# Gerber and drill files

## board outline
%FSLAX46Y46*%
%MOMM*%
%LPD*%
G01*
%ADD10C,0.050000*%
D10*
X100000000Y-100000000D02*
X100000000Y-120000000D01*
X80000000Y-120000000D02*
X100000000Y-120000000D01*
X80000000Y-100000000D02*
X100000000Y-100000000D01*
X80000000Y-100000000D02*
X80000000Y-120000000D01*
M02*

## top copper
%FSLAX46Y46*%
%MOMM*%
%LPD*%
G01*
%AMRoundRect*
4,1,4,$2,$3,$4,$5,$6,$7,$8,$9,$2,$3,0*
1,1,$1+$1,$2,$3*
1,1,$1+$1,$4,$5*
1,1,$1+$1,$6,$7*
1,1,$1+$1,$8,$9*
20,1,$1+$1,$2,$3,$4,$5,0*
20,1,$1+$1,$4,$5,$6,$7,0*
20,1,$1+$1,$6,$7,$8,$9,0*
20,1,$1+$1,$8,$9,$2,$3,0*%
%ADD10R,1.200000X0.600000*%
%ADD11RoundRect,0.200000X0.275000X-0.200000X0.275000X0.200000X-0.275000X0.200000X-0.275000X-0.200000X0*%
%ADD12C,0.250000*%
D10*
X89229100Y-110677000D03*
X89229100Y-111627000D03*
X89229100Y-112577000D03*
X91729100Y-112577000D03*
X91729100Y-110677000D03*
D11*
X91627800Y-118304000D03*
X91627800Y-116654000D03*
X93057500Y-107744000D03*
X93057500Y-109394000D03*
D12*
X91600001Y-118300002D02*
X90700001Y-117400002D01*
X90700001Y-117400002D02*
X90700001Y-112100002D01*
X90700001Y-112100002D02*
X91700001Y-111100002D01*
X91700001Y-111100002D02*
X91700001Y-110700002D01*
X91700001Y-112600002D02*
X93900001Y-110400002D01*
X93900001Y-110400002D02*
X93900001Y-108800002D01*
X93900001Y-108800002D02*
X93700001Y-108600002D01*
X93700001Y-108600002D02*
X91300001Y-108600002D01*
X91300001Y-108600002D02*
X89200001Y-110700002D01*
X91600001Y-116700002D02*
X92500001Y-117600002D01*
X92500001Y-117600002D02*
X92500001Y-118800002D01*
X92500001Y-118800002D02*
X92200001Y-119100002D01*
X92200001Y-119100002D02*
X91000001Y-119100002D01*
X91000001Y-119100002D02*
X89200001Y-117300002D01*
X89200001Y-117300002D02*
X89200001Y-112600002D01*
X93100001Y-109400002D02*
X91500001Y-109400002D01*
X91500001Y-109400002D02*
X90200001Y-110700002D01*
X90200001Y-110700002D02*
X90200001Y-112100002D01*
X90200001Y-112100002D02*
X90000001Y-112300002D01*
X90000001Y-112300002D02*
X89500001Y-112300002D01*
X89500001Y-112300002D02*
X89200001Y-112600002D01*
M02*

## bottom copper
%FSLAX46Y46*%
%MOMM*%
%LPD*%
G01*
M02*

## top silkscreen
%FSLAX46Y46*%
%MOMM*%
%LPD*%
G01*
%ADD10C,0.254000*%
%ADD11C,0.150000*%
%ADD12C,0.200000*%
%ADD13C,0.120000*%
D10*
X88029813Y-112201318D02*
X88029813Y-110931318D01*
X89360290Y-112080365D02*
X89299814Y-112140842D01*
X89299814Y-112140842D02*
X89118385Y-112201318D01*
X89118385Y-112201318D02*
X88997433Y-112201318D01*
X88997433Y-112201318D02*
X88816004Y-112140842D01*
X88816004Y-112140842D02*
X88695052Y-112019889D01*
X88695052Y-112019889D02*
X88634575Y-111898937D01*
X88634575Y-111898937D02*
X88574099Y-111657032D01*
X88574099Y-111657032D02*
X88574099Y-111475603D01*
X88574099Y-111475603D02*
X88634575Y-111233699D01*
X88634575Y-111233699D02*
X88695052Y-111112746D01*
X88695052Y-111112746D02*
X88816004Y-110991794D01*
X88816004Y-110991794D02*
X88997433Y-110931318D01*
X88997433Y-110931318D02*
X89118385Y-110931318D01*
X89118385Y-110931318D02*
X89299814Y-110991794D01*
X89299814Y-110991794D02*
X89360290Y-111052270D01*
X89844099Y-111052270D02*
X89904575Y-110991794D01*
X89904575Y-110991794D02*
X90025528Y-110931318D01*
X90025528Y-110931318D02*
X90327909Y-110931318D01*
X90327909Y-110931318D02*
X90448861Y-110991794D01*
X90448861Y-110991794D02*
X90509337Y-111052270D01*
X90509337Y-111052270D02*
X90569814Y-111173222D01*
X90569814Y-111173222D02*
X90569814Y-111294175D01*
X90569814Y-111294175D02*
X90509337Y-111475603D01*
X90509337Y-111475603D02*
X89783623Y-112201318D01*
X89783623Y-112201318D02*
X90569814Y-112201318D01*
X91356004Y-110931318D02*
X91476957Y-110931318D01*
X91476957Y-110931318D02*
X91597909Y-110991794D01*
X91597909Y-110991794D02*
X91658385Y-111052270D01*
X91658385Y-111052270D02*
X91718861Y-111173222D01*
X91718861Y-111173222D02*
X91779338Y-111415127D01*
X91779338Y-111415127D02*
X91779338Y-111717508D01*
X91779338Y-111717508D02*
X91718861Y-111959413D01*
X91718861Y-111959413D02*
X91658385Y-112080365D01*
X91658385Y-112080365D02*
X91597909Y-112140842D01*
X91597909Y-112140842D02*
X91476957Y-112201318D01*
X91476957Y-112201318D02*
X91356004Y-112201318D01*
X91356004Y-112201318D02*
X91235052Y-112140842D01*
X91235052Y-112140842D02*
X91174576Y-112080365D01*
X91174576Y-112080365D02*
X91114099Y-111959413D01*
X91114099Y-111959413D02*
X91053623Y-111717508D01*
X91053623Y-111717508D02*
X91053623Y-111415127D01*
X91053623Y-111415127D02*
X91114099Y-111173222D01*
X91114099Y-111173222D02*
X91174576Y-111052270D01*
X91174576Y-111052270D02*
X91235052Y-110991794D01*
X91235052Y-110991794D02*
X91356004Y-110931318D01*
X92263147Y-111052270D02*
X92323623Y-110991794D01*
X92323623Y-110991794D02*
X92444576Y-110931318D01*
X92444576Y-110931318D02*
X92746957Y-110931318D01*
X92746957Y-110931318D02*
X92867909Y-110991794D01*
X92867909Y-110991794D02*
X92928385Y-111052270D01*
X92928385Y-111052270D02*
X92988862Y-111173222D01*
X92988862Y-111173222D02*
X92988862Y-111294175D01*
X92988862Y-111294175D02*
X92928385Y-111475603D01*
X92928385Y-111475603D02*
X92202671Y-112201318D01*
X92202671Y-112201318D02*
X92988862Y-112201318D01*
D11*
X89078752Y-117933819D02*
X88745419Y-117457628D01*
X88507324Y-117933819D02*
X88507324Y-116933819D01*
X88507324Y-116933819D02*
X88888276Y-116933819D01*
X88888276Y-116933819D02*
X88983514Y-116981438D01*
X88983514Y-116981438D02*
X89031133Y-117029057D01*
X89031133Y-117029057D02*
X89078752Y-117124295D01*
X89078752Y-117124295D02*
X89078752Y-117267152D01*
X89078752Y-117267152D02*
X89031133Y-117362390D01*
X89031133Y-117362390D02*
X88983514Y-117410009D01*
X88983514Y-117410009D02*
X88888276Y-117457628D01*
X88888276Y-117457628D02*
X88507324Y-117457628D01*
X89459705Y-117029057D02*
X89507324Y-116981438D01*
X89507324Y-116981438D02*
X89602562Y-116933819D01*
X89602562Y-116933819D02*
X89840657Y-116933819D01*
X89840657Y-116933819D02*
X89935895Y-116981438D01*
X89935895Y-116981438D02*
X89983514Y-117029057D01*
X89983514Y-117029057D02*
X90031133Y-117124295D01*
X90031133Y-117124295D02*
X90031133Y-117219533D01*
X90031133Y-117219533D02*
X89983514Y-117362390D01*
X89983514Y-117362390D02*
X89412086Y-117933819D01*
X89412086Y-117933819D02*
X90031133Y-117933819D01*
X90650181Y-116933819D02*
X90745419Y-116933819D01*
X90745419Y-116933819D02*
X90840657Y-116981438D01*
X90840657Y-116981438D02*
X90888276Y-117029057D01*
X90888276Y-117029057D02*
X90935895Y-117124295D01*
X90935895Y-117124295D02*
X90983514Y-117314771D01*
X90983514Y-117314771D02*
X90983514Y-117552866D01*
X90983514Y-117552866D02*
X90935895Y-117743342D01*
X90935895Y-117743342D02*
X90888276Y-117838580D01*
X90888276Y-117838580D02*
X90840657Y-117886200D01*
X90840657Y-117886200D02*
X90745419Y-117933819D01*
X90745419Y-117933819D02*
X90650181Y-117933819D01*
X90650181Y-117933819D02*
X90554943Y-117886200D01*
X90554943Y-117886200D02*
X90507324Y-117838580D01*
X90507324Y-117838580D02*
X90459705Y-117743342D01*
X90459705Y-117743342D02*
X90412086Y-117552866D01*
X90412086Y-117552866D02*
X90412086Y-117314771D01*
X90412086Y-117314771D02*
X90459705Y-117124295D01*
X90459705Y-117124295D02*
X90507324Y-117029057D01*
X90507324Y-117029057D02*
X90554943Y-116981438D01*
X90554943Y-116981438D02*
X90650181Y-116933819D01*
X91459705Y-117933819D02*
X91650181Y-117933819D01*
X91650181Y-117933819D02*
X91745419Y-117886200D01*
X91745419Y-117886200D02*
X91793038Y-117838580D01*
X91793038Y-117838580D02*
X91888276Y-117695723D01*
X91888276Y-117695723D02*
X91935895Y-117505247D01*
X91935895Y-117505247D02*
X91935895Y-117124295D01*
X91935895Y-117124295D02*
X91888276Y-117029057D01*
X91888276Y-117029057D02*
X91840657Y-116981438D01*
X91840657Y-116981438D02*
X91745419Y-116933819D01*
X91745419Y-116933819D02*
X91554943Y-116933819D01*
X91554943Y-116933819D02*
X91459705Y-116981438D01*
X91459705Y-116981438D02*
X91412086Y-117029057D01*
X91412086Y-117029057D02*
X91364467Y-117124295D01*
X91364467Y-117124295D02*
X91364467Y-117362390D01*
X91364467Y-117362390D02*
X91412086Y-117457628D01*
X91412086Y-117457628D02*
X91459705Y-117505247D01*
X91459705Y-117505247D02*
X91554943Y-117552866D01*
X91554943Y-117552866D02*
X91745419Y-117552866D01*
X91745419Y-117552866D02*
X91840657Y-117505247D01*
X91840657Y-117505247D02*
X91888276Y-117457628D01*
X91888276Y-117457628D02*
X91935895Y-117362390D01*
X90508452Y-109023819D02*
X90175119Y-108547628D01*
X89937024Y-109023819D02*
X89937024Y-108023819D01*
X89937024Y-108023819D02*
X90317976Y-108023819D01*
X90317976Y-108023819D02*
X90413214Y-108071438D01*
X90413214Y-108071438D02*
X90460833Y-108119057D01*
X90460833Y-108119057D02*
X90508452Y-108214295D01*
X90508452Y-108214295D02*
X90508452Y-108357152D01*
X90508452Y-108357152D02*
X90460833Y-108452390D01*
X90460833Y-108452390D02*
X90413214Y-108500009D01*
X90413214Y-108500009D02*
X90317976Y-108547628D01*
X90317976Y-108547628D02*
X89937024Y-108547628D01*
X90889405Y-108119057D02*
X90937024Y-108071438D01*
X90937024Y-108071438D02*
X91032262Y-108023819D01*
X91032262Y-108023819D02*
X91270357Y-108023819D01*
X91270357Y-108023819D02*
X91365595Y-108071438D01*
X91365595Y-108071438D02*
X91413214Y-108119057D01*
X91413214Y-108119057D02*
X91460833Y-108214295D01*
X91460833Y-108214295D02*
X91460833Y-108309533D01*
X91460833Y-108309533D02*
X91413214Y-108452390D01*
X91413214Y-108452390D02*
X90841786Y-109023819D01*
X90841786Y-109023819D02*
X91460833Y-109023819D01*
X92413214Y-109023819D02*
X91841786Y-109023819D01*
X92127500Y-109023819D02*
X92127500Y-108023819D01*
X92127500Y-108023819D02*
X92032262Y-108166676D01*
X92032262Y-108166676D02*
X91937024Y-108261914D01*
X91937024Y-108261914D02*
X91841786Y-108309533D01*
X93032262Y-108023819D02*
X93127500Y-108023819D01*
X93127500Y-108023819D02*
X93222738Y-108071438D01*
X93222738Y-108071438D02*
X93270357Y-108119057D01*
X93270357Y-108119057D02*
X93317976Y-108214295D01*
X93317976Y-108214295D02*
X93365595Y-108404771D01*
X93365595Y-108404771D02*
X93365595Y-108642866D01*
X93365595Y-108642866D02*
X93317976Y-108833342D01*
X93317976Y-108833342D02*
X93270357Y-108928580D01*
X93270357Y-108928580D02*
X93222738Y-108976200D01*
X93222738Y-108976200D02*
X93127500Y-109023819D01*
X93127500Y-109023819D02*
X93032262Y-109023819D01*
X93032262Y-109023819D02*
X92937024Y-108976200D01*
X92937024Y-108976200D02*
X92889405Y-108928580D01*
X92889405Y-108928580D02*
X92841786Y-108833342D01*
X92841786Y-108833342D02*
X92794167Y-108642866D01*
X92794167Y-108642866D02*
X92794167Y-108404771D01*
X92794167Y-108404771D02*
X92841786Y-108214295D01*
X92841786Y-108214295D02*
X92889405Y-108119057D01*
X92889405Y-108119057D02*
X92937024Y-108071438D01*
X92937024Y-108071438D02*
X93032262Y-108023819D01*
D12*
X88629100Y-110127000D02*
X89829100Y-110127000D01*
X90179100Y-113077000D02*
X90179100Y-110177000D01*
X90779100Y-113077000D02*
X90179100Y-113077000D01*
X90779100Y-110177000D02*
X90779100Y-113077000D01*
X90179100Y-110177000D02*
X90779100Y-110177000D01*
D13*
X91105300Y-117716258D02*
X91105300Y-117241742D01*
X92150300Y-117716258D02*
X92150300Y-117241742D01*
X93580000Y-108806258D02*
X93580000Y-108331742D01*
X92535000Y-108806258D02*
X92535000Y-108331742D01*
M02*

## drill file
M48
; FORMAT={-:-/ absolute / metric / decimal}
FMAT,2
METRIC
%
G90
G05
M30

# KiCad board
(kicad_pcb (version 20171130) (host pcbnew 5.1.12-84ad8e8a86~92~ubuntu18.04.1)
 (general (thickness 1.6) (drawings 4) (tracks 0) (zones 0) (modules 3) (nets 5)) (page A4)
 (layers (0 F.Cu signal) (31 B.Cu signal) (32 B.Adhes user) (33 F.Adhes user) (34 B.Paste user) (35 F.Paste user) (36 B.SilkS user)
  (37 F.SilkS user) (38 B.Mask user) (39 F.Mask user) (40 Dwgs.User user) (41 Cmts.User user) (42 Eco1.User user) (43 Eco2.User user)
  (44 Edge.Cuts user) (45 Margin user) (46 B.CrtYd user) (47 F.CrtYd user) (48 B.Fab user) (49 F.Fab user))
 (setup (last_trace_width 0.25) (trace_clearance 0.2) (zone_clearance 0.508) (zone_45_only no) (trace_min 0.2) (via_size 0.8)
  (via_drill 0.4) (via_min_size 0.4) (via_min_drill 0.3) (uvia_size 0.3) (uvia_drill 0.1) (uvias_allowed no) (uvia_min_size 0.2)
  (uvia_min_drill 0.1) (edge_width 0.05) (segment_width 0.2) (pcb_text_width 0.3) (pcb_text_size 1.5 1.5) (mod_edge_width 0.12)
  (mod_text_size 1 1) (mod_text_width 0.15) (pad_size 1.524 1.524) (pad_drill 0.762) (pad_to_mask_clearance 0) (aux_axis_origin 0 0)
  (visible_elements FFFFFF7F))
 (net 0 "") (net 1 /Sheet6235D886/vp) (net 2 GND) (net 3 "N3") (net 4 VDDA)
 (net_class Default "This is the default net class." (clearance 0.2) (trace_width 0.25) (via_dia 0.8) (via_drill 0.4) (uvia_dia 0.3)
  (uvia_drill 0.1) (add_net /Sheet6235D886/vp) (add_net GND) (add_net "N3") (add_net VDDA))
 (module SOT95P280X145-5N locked (layer F.Cu) (at 90.479100 111.627000)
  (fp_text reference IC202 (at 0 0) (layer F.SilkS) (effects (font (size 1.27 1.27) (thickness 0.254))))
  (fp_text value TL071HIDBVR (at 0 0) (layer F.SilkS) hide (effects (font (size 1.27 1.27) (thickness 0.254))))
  (fp_line (start -1.85 -1.5) (end -0.65 -1.5) (layer F.SilkS) (width 0.2))
  (fp_line (start -0.3 1.45) (end -0.3 -1.45) (layer F.SilkS) (width 0.2))
  (fp_line (start 0.3 1.45) (end -0.3 1.45) (layer F.SilkS) (width 0.2))
  (fp_line (start 0.3 -1.45) (end 0.3 1.45) (layer F.SilkS) (width 0.2))
  (fp_line (start -0.3 -1.45) (end 0.3 -1.45) (layer F.SilkS) (width 0.2))
  (pad 1 smd rect (at -1.25 -0.95 90.000000) (size 0.6 1.2) (layers F.Cu F.Mask F.Paste) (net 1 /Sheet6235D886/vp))
  (pad 2 smd rect (at -1.25 0 90.000000) (size 0.6 1.2) (layers F.Cu F.Mask F.Paste) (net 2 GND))
  (pad 3 smd rect (at -1.25 0.95 90.000000) (size 0.6 1.2) (layers F.Cu F.Mask F.Paste) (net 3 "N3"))
  (pad 4 smd rect (at 1.25 0.95 90.000000) (size 0.6 1.2) (layers F.Cu F.Mask F.Paste) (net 1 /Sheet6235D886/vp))
  (pad 5 smd rect (at 1.25 -0.95 90.000000) (size 0.6 1.2) (layers F.Cu F.Mask F.Paste) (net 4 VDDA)))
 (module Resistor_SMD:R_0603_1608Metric (layer F.Cu) (at 91.627800 117.479000 90.000000)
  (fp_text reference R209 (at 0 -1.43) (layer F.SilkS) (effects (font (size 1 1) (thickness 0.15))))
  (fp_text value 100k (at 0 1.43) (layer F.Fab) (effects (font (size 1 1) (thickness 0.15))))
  (fp_line (start -0.237258 -0.5225) (end 0.237258 -0.5225) (layer F.SilkS) (width 0.12))
  (fp_line (start -0.237258 0.5225) (end 0.237258 0.5225) (layer F.SilkS) (width 0.12))
  (pad 1 smd roundrect (at -0.825 0 90.000000) (size 0.8 0.95) (layers F.Cu F.Mask F.Paste) (roundrect_rratio 0.25) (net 4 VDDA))
  (pad 2 smd roundrect (at 0.825 0 90.000000) (size 0.8 0.95) (layers F.Cu F.Mask F.Paste) (roundrect_rratio 0.25) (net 3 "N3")))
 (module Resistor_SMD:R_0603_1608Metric (layer F.Cu) (at 93.057500 108.569000 90.000000)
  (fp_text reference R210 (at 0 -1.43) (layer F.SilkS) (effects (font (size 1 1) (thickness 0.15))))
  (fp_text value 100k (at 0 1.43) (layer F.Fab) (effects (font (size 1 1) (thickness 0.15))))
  (fp_line (start -0.237258 0.5225) (end 0.237258 0.5225) (layer F.SilkS) (width 0.12))
  (fp_line (start -0.237258 -0.5225) (end 0.237258 -0.5225) (layer F.SilkS) (width 0.12))
  (pad 2 smd roundrect (at 0.825 0 90.000000) (size 0.8 0.95) (layers F.Cu F.Mask F.Paste) (roundrect_rratio 0.25) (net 2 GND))
  (pad 1 smd roundrect (at -0.825 0 90.000000) (size 0.8 0.95) (layers F.Cu F.Mask F.Paste) (roundrect_rratio 0.25) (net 3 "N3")))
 (gr_line (start 100 100) (end 100 120) (layer Edge.Cuts) (width 0.05))
 (gr_line (start 80 120) (end 100 120) (layer Edge.Cuts) (width 0.05))
 (gr_line (start 80 100) (end 100 100) (layer Edge.Cuts) (width 0.05))
 (gr_line (start 80 100) (end 80 120) (layer Edge.Cuts) (width 0.05))
 (segment (start 91.600001 118.300002) (end 90.700001 117.400002) (width 0.250000) (layer F.Cu) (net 4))
 (segment (start 90.700001 117.400002) (end 90.700001 112.100002) (width 0.250000) (layer F.Cu) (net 4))
 (segment (start 90.700001 112.100002) (end 91.700001 111.100002) (width 0.250000) (layer F.Cu) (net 4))
 (segment (start 91.700001 111.100002) (end 91.700001 110.700002) (width 0.250000) (layer F.Cu) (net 4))
 (segment (start 91.700001 112.600002) (end 93.900001 110.400002) (width 0.250000) (layer F.Cu) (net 1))
 (segment (start 93.900001 110.400002) (end 93.900001 108.800002) (width 0.250000) (layer F.Cu) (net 1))
 (segment (start 93.900001 108.800002) (end 93.700001 108.600002) (width 0.250000) (layer F.Cu) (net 1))
 (segment (start 93.700001 108.600002) (end 91.300001 108.600002) (width 0.250000) (layer F.Cu) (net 1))
 (segment (start 91.300001 108.600002) (end 89.200001 110.700002) (width 0.250000) (layer F.Cu) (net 1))
 (segment (start 91.600001 116.700002) (end 92.500001 117.600002) (width 0.250000) (layer F.Cu) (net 3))
 (segment (start 92.500001 117.600002) (end 92.500001 118.800002) (width 0.250000) (layer F.Cu) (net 3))
 (segment (start 92.500001 118.800002) (end 92.200001 119.100002) (width 0.250000) (layer F.Cu) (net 3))
 (segment (start 92.200001 119.100002) (end 91.000001 119.100002) (width 0.250000) (layer F.Cu) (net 3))
 (segment (start 91.000001 119.100002) (end 89.200001 117.300002) (width 0.250000) (layer F.Cu) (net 3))
 (segment (start 89.200001 117.300002) (end 89.200001 112.600002) (width 0.250000) (layer F.Cu) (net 3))
 (segment (start 93.100001 109.400002) (end 91.500001 109.400002) (width 0.250000) (layer F.Cu) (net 3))
 (segment (start 91.500001 109.400002) (end 90.200001 110.700002) (width 0.250000) (layer F.Cu) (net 3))
 (segment (start 90.200001 110.700002) (end 90.200001 112.100002) (width 0.250000) (layer F.Cu) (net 3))
 (segment (start 90.200001 112.100002) (end 90.000001 112.300002) (width 0.250000) (layer F.Cu) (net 3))
 (segment (start 90.000001 112.300002) (end 89.500001 112.300002) (width 0.250000) (layer F.Cu) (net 3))
 (segment (start 89.500001 112.300002) (end 89.200001 112.600002) (width 0.250000) (layer F.Cu) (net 3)))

